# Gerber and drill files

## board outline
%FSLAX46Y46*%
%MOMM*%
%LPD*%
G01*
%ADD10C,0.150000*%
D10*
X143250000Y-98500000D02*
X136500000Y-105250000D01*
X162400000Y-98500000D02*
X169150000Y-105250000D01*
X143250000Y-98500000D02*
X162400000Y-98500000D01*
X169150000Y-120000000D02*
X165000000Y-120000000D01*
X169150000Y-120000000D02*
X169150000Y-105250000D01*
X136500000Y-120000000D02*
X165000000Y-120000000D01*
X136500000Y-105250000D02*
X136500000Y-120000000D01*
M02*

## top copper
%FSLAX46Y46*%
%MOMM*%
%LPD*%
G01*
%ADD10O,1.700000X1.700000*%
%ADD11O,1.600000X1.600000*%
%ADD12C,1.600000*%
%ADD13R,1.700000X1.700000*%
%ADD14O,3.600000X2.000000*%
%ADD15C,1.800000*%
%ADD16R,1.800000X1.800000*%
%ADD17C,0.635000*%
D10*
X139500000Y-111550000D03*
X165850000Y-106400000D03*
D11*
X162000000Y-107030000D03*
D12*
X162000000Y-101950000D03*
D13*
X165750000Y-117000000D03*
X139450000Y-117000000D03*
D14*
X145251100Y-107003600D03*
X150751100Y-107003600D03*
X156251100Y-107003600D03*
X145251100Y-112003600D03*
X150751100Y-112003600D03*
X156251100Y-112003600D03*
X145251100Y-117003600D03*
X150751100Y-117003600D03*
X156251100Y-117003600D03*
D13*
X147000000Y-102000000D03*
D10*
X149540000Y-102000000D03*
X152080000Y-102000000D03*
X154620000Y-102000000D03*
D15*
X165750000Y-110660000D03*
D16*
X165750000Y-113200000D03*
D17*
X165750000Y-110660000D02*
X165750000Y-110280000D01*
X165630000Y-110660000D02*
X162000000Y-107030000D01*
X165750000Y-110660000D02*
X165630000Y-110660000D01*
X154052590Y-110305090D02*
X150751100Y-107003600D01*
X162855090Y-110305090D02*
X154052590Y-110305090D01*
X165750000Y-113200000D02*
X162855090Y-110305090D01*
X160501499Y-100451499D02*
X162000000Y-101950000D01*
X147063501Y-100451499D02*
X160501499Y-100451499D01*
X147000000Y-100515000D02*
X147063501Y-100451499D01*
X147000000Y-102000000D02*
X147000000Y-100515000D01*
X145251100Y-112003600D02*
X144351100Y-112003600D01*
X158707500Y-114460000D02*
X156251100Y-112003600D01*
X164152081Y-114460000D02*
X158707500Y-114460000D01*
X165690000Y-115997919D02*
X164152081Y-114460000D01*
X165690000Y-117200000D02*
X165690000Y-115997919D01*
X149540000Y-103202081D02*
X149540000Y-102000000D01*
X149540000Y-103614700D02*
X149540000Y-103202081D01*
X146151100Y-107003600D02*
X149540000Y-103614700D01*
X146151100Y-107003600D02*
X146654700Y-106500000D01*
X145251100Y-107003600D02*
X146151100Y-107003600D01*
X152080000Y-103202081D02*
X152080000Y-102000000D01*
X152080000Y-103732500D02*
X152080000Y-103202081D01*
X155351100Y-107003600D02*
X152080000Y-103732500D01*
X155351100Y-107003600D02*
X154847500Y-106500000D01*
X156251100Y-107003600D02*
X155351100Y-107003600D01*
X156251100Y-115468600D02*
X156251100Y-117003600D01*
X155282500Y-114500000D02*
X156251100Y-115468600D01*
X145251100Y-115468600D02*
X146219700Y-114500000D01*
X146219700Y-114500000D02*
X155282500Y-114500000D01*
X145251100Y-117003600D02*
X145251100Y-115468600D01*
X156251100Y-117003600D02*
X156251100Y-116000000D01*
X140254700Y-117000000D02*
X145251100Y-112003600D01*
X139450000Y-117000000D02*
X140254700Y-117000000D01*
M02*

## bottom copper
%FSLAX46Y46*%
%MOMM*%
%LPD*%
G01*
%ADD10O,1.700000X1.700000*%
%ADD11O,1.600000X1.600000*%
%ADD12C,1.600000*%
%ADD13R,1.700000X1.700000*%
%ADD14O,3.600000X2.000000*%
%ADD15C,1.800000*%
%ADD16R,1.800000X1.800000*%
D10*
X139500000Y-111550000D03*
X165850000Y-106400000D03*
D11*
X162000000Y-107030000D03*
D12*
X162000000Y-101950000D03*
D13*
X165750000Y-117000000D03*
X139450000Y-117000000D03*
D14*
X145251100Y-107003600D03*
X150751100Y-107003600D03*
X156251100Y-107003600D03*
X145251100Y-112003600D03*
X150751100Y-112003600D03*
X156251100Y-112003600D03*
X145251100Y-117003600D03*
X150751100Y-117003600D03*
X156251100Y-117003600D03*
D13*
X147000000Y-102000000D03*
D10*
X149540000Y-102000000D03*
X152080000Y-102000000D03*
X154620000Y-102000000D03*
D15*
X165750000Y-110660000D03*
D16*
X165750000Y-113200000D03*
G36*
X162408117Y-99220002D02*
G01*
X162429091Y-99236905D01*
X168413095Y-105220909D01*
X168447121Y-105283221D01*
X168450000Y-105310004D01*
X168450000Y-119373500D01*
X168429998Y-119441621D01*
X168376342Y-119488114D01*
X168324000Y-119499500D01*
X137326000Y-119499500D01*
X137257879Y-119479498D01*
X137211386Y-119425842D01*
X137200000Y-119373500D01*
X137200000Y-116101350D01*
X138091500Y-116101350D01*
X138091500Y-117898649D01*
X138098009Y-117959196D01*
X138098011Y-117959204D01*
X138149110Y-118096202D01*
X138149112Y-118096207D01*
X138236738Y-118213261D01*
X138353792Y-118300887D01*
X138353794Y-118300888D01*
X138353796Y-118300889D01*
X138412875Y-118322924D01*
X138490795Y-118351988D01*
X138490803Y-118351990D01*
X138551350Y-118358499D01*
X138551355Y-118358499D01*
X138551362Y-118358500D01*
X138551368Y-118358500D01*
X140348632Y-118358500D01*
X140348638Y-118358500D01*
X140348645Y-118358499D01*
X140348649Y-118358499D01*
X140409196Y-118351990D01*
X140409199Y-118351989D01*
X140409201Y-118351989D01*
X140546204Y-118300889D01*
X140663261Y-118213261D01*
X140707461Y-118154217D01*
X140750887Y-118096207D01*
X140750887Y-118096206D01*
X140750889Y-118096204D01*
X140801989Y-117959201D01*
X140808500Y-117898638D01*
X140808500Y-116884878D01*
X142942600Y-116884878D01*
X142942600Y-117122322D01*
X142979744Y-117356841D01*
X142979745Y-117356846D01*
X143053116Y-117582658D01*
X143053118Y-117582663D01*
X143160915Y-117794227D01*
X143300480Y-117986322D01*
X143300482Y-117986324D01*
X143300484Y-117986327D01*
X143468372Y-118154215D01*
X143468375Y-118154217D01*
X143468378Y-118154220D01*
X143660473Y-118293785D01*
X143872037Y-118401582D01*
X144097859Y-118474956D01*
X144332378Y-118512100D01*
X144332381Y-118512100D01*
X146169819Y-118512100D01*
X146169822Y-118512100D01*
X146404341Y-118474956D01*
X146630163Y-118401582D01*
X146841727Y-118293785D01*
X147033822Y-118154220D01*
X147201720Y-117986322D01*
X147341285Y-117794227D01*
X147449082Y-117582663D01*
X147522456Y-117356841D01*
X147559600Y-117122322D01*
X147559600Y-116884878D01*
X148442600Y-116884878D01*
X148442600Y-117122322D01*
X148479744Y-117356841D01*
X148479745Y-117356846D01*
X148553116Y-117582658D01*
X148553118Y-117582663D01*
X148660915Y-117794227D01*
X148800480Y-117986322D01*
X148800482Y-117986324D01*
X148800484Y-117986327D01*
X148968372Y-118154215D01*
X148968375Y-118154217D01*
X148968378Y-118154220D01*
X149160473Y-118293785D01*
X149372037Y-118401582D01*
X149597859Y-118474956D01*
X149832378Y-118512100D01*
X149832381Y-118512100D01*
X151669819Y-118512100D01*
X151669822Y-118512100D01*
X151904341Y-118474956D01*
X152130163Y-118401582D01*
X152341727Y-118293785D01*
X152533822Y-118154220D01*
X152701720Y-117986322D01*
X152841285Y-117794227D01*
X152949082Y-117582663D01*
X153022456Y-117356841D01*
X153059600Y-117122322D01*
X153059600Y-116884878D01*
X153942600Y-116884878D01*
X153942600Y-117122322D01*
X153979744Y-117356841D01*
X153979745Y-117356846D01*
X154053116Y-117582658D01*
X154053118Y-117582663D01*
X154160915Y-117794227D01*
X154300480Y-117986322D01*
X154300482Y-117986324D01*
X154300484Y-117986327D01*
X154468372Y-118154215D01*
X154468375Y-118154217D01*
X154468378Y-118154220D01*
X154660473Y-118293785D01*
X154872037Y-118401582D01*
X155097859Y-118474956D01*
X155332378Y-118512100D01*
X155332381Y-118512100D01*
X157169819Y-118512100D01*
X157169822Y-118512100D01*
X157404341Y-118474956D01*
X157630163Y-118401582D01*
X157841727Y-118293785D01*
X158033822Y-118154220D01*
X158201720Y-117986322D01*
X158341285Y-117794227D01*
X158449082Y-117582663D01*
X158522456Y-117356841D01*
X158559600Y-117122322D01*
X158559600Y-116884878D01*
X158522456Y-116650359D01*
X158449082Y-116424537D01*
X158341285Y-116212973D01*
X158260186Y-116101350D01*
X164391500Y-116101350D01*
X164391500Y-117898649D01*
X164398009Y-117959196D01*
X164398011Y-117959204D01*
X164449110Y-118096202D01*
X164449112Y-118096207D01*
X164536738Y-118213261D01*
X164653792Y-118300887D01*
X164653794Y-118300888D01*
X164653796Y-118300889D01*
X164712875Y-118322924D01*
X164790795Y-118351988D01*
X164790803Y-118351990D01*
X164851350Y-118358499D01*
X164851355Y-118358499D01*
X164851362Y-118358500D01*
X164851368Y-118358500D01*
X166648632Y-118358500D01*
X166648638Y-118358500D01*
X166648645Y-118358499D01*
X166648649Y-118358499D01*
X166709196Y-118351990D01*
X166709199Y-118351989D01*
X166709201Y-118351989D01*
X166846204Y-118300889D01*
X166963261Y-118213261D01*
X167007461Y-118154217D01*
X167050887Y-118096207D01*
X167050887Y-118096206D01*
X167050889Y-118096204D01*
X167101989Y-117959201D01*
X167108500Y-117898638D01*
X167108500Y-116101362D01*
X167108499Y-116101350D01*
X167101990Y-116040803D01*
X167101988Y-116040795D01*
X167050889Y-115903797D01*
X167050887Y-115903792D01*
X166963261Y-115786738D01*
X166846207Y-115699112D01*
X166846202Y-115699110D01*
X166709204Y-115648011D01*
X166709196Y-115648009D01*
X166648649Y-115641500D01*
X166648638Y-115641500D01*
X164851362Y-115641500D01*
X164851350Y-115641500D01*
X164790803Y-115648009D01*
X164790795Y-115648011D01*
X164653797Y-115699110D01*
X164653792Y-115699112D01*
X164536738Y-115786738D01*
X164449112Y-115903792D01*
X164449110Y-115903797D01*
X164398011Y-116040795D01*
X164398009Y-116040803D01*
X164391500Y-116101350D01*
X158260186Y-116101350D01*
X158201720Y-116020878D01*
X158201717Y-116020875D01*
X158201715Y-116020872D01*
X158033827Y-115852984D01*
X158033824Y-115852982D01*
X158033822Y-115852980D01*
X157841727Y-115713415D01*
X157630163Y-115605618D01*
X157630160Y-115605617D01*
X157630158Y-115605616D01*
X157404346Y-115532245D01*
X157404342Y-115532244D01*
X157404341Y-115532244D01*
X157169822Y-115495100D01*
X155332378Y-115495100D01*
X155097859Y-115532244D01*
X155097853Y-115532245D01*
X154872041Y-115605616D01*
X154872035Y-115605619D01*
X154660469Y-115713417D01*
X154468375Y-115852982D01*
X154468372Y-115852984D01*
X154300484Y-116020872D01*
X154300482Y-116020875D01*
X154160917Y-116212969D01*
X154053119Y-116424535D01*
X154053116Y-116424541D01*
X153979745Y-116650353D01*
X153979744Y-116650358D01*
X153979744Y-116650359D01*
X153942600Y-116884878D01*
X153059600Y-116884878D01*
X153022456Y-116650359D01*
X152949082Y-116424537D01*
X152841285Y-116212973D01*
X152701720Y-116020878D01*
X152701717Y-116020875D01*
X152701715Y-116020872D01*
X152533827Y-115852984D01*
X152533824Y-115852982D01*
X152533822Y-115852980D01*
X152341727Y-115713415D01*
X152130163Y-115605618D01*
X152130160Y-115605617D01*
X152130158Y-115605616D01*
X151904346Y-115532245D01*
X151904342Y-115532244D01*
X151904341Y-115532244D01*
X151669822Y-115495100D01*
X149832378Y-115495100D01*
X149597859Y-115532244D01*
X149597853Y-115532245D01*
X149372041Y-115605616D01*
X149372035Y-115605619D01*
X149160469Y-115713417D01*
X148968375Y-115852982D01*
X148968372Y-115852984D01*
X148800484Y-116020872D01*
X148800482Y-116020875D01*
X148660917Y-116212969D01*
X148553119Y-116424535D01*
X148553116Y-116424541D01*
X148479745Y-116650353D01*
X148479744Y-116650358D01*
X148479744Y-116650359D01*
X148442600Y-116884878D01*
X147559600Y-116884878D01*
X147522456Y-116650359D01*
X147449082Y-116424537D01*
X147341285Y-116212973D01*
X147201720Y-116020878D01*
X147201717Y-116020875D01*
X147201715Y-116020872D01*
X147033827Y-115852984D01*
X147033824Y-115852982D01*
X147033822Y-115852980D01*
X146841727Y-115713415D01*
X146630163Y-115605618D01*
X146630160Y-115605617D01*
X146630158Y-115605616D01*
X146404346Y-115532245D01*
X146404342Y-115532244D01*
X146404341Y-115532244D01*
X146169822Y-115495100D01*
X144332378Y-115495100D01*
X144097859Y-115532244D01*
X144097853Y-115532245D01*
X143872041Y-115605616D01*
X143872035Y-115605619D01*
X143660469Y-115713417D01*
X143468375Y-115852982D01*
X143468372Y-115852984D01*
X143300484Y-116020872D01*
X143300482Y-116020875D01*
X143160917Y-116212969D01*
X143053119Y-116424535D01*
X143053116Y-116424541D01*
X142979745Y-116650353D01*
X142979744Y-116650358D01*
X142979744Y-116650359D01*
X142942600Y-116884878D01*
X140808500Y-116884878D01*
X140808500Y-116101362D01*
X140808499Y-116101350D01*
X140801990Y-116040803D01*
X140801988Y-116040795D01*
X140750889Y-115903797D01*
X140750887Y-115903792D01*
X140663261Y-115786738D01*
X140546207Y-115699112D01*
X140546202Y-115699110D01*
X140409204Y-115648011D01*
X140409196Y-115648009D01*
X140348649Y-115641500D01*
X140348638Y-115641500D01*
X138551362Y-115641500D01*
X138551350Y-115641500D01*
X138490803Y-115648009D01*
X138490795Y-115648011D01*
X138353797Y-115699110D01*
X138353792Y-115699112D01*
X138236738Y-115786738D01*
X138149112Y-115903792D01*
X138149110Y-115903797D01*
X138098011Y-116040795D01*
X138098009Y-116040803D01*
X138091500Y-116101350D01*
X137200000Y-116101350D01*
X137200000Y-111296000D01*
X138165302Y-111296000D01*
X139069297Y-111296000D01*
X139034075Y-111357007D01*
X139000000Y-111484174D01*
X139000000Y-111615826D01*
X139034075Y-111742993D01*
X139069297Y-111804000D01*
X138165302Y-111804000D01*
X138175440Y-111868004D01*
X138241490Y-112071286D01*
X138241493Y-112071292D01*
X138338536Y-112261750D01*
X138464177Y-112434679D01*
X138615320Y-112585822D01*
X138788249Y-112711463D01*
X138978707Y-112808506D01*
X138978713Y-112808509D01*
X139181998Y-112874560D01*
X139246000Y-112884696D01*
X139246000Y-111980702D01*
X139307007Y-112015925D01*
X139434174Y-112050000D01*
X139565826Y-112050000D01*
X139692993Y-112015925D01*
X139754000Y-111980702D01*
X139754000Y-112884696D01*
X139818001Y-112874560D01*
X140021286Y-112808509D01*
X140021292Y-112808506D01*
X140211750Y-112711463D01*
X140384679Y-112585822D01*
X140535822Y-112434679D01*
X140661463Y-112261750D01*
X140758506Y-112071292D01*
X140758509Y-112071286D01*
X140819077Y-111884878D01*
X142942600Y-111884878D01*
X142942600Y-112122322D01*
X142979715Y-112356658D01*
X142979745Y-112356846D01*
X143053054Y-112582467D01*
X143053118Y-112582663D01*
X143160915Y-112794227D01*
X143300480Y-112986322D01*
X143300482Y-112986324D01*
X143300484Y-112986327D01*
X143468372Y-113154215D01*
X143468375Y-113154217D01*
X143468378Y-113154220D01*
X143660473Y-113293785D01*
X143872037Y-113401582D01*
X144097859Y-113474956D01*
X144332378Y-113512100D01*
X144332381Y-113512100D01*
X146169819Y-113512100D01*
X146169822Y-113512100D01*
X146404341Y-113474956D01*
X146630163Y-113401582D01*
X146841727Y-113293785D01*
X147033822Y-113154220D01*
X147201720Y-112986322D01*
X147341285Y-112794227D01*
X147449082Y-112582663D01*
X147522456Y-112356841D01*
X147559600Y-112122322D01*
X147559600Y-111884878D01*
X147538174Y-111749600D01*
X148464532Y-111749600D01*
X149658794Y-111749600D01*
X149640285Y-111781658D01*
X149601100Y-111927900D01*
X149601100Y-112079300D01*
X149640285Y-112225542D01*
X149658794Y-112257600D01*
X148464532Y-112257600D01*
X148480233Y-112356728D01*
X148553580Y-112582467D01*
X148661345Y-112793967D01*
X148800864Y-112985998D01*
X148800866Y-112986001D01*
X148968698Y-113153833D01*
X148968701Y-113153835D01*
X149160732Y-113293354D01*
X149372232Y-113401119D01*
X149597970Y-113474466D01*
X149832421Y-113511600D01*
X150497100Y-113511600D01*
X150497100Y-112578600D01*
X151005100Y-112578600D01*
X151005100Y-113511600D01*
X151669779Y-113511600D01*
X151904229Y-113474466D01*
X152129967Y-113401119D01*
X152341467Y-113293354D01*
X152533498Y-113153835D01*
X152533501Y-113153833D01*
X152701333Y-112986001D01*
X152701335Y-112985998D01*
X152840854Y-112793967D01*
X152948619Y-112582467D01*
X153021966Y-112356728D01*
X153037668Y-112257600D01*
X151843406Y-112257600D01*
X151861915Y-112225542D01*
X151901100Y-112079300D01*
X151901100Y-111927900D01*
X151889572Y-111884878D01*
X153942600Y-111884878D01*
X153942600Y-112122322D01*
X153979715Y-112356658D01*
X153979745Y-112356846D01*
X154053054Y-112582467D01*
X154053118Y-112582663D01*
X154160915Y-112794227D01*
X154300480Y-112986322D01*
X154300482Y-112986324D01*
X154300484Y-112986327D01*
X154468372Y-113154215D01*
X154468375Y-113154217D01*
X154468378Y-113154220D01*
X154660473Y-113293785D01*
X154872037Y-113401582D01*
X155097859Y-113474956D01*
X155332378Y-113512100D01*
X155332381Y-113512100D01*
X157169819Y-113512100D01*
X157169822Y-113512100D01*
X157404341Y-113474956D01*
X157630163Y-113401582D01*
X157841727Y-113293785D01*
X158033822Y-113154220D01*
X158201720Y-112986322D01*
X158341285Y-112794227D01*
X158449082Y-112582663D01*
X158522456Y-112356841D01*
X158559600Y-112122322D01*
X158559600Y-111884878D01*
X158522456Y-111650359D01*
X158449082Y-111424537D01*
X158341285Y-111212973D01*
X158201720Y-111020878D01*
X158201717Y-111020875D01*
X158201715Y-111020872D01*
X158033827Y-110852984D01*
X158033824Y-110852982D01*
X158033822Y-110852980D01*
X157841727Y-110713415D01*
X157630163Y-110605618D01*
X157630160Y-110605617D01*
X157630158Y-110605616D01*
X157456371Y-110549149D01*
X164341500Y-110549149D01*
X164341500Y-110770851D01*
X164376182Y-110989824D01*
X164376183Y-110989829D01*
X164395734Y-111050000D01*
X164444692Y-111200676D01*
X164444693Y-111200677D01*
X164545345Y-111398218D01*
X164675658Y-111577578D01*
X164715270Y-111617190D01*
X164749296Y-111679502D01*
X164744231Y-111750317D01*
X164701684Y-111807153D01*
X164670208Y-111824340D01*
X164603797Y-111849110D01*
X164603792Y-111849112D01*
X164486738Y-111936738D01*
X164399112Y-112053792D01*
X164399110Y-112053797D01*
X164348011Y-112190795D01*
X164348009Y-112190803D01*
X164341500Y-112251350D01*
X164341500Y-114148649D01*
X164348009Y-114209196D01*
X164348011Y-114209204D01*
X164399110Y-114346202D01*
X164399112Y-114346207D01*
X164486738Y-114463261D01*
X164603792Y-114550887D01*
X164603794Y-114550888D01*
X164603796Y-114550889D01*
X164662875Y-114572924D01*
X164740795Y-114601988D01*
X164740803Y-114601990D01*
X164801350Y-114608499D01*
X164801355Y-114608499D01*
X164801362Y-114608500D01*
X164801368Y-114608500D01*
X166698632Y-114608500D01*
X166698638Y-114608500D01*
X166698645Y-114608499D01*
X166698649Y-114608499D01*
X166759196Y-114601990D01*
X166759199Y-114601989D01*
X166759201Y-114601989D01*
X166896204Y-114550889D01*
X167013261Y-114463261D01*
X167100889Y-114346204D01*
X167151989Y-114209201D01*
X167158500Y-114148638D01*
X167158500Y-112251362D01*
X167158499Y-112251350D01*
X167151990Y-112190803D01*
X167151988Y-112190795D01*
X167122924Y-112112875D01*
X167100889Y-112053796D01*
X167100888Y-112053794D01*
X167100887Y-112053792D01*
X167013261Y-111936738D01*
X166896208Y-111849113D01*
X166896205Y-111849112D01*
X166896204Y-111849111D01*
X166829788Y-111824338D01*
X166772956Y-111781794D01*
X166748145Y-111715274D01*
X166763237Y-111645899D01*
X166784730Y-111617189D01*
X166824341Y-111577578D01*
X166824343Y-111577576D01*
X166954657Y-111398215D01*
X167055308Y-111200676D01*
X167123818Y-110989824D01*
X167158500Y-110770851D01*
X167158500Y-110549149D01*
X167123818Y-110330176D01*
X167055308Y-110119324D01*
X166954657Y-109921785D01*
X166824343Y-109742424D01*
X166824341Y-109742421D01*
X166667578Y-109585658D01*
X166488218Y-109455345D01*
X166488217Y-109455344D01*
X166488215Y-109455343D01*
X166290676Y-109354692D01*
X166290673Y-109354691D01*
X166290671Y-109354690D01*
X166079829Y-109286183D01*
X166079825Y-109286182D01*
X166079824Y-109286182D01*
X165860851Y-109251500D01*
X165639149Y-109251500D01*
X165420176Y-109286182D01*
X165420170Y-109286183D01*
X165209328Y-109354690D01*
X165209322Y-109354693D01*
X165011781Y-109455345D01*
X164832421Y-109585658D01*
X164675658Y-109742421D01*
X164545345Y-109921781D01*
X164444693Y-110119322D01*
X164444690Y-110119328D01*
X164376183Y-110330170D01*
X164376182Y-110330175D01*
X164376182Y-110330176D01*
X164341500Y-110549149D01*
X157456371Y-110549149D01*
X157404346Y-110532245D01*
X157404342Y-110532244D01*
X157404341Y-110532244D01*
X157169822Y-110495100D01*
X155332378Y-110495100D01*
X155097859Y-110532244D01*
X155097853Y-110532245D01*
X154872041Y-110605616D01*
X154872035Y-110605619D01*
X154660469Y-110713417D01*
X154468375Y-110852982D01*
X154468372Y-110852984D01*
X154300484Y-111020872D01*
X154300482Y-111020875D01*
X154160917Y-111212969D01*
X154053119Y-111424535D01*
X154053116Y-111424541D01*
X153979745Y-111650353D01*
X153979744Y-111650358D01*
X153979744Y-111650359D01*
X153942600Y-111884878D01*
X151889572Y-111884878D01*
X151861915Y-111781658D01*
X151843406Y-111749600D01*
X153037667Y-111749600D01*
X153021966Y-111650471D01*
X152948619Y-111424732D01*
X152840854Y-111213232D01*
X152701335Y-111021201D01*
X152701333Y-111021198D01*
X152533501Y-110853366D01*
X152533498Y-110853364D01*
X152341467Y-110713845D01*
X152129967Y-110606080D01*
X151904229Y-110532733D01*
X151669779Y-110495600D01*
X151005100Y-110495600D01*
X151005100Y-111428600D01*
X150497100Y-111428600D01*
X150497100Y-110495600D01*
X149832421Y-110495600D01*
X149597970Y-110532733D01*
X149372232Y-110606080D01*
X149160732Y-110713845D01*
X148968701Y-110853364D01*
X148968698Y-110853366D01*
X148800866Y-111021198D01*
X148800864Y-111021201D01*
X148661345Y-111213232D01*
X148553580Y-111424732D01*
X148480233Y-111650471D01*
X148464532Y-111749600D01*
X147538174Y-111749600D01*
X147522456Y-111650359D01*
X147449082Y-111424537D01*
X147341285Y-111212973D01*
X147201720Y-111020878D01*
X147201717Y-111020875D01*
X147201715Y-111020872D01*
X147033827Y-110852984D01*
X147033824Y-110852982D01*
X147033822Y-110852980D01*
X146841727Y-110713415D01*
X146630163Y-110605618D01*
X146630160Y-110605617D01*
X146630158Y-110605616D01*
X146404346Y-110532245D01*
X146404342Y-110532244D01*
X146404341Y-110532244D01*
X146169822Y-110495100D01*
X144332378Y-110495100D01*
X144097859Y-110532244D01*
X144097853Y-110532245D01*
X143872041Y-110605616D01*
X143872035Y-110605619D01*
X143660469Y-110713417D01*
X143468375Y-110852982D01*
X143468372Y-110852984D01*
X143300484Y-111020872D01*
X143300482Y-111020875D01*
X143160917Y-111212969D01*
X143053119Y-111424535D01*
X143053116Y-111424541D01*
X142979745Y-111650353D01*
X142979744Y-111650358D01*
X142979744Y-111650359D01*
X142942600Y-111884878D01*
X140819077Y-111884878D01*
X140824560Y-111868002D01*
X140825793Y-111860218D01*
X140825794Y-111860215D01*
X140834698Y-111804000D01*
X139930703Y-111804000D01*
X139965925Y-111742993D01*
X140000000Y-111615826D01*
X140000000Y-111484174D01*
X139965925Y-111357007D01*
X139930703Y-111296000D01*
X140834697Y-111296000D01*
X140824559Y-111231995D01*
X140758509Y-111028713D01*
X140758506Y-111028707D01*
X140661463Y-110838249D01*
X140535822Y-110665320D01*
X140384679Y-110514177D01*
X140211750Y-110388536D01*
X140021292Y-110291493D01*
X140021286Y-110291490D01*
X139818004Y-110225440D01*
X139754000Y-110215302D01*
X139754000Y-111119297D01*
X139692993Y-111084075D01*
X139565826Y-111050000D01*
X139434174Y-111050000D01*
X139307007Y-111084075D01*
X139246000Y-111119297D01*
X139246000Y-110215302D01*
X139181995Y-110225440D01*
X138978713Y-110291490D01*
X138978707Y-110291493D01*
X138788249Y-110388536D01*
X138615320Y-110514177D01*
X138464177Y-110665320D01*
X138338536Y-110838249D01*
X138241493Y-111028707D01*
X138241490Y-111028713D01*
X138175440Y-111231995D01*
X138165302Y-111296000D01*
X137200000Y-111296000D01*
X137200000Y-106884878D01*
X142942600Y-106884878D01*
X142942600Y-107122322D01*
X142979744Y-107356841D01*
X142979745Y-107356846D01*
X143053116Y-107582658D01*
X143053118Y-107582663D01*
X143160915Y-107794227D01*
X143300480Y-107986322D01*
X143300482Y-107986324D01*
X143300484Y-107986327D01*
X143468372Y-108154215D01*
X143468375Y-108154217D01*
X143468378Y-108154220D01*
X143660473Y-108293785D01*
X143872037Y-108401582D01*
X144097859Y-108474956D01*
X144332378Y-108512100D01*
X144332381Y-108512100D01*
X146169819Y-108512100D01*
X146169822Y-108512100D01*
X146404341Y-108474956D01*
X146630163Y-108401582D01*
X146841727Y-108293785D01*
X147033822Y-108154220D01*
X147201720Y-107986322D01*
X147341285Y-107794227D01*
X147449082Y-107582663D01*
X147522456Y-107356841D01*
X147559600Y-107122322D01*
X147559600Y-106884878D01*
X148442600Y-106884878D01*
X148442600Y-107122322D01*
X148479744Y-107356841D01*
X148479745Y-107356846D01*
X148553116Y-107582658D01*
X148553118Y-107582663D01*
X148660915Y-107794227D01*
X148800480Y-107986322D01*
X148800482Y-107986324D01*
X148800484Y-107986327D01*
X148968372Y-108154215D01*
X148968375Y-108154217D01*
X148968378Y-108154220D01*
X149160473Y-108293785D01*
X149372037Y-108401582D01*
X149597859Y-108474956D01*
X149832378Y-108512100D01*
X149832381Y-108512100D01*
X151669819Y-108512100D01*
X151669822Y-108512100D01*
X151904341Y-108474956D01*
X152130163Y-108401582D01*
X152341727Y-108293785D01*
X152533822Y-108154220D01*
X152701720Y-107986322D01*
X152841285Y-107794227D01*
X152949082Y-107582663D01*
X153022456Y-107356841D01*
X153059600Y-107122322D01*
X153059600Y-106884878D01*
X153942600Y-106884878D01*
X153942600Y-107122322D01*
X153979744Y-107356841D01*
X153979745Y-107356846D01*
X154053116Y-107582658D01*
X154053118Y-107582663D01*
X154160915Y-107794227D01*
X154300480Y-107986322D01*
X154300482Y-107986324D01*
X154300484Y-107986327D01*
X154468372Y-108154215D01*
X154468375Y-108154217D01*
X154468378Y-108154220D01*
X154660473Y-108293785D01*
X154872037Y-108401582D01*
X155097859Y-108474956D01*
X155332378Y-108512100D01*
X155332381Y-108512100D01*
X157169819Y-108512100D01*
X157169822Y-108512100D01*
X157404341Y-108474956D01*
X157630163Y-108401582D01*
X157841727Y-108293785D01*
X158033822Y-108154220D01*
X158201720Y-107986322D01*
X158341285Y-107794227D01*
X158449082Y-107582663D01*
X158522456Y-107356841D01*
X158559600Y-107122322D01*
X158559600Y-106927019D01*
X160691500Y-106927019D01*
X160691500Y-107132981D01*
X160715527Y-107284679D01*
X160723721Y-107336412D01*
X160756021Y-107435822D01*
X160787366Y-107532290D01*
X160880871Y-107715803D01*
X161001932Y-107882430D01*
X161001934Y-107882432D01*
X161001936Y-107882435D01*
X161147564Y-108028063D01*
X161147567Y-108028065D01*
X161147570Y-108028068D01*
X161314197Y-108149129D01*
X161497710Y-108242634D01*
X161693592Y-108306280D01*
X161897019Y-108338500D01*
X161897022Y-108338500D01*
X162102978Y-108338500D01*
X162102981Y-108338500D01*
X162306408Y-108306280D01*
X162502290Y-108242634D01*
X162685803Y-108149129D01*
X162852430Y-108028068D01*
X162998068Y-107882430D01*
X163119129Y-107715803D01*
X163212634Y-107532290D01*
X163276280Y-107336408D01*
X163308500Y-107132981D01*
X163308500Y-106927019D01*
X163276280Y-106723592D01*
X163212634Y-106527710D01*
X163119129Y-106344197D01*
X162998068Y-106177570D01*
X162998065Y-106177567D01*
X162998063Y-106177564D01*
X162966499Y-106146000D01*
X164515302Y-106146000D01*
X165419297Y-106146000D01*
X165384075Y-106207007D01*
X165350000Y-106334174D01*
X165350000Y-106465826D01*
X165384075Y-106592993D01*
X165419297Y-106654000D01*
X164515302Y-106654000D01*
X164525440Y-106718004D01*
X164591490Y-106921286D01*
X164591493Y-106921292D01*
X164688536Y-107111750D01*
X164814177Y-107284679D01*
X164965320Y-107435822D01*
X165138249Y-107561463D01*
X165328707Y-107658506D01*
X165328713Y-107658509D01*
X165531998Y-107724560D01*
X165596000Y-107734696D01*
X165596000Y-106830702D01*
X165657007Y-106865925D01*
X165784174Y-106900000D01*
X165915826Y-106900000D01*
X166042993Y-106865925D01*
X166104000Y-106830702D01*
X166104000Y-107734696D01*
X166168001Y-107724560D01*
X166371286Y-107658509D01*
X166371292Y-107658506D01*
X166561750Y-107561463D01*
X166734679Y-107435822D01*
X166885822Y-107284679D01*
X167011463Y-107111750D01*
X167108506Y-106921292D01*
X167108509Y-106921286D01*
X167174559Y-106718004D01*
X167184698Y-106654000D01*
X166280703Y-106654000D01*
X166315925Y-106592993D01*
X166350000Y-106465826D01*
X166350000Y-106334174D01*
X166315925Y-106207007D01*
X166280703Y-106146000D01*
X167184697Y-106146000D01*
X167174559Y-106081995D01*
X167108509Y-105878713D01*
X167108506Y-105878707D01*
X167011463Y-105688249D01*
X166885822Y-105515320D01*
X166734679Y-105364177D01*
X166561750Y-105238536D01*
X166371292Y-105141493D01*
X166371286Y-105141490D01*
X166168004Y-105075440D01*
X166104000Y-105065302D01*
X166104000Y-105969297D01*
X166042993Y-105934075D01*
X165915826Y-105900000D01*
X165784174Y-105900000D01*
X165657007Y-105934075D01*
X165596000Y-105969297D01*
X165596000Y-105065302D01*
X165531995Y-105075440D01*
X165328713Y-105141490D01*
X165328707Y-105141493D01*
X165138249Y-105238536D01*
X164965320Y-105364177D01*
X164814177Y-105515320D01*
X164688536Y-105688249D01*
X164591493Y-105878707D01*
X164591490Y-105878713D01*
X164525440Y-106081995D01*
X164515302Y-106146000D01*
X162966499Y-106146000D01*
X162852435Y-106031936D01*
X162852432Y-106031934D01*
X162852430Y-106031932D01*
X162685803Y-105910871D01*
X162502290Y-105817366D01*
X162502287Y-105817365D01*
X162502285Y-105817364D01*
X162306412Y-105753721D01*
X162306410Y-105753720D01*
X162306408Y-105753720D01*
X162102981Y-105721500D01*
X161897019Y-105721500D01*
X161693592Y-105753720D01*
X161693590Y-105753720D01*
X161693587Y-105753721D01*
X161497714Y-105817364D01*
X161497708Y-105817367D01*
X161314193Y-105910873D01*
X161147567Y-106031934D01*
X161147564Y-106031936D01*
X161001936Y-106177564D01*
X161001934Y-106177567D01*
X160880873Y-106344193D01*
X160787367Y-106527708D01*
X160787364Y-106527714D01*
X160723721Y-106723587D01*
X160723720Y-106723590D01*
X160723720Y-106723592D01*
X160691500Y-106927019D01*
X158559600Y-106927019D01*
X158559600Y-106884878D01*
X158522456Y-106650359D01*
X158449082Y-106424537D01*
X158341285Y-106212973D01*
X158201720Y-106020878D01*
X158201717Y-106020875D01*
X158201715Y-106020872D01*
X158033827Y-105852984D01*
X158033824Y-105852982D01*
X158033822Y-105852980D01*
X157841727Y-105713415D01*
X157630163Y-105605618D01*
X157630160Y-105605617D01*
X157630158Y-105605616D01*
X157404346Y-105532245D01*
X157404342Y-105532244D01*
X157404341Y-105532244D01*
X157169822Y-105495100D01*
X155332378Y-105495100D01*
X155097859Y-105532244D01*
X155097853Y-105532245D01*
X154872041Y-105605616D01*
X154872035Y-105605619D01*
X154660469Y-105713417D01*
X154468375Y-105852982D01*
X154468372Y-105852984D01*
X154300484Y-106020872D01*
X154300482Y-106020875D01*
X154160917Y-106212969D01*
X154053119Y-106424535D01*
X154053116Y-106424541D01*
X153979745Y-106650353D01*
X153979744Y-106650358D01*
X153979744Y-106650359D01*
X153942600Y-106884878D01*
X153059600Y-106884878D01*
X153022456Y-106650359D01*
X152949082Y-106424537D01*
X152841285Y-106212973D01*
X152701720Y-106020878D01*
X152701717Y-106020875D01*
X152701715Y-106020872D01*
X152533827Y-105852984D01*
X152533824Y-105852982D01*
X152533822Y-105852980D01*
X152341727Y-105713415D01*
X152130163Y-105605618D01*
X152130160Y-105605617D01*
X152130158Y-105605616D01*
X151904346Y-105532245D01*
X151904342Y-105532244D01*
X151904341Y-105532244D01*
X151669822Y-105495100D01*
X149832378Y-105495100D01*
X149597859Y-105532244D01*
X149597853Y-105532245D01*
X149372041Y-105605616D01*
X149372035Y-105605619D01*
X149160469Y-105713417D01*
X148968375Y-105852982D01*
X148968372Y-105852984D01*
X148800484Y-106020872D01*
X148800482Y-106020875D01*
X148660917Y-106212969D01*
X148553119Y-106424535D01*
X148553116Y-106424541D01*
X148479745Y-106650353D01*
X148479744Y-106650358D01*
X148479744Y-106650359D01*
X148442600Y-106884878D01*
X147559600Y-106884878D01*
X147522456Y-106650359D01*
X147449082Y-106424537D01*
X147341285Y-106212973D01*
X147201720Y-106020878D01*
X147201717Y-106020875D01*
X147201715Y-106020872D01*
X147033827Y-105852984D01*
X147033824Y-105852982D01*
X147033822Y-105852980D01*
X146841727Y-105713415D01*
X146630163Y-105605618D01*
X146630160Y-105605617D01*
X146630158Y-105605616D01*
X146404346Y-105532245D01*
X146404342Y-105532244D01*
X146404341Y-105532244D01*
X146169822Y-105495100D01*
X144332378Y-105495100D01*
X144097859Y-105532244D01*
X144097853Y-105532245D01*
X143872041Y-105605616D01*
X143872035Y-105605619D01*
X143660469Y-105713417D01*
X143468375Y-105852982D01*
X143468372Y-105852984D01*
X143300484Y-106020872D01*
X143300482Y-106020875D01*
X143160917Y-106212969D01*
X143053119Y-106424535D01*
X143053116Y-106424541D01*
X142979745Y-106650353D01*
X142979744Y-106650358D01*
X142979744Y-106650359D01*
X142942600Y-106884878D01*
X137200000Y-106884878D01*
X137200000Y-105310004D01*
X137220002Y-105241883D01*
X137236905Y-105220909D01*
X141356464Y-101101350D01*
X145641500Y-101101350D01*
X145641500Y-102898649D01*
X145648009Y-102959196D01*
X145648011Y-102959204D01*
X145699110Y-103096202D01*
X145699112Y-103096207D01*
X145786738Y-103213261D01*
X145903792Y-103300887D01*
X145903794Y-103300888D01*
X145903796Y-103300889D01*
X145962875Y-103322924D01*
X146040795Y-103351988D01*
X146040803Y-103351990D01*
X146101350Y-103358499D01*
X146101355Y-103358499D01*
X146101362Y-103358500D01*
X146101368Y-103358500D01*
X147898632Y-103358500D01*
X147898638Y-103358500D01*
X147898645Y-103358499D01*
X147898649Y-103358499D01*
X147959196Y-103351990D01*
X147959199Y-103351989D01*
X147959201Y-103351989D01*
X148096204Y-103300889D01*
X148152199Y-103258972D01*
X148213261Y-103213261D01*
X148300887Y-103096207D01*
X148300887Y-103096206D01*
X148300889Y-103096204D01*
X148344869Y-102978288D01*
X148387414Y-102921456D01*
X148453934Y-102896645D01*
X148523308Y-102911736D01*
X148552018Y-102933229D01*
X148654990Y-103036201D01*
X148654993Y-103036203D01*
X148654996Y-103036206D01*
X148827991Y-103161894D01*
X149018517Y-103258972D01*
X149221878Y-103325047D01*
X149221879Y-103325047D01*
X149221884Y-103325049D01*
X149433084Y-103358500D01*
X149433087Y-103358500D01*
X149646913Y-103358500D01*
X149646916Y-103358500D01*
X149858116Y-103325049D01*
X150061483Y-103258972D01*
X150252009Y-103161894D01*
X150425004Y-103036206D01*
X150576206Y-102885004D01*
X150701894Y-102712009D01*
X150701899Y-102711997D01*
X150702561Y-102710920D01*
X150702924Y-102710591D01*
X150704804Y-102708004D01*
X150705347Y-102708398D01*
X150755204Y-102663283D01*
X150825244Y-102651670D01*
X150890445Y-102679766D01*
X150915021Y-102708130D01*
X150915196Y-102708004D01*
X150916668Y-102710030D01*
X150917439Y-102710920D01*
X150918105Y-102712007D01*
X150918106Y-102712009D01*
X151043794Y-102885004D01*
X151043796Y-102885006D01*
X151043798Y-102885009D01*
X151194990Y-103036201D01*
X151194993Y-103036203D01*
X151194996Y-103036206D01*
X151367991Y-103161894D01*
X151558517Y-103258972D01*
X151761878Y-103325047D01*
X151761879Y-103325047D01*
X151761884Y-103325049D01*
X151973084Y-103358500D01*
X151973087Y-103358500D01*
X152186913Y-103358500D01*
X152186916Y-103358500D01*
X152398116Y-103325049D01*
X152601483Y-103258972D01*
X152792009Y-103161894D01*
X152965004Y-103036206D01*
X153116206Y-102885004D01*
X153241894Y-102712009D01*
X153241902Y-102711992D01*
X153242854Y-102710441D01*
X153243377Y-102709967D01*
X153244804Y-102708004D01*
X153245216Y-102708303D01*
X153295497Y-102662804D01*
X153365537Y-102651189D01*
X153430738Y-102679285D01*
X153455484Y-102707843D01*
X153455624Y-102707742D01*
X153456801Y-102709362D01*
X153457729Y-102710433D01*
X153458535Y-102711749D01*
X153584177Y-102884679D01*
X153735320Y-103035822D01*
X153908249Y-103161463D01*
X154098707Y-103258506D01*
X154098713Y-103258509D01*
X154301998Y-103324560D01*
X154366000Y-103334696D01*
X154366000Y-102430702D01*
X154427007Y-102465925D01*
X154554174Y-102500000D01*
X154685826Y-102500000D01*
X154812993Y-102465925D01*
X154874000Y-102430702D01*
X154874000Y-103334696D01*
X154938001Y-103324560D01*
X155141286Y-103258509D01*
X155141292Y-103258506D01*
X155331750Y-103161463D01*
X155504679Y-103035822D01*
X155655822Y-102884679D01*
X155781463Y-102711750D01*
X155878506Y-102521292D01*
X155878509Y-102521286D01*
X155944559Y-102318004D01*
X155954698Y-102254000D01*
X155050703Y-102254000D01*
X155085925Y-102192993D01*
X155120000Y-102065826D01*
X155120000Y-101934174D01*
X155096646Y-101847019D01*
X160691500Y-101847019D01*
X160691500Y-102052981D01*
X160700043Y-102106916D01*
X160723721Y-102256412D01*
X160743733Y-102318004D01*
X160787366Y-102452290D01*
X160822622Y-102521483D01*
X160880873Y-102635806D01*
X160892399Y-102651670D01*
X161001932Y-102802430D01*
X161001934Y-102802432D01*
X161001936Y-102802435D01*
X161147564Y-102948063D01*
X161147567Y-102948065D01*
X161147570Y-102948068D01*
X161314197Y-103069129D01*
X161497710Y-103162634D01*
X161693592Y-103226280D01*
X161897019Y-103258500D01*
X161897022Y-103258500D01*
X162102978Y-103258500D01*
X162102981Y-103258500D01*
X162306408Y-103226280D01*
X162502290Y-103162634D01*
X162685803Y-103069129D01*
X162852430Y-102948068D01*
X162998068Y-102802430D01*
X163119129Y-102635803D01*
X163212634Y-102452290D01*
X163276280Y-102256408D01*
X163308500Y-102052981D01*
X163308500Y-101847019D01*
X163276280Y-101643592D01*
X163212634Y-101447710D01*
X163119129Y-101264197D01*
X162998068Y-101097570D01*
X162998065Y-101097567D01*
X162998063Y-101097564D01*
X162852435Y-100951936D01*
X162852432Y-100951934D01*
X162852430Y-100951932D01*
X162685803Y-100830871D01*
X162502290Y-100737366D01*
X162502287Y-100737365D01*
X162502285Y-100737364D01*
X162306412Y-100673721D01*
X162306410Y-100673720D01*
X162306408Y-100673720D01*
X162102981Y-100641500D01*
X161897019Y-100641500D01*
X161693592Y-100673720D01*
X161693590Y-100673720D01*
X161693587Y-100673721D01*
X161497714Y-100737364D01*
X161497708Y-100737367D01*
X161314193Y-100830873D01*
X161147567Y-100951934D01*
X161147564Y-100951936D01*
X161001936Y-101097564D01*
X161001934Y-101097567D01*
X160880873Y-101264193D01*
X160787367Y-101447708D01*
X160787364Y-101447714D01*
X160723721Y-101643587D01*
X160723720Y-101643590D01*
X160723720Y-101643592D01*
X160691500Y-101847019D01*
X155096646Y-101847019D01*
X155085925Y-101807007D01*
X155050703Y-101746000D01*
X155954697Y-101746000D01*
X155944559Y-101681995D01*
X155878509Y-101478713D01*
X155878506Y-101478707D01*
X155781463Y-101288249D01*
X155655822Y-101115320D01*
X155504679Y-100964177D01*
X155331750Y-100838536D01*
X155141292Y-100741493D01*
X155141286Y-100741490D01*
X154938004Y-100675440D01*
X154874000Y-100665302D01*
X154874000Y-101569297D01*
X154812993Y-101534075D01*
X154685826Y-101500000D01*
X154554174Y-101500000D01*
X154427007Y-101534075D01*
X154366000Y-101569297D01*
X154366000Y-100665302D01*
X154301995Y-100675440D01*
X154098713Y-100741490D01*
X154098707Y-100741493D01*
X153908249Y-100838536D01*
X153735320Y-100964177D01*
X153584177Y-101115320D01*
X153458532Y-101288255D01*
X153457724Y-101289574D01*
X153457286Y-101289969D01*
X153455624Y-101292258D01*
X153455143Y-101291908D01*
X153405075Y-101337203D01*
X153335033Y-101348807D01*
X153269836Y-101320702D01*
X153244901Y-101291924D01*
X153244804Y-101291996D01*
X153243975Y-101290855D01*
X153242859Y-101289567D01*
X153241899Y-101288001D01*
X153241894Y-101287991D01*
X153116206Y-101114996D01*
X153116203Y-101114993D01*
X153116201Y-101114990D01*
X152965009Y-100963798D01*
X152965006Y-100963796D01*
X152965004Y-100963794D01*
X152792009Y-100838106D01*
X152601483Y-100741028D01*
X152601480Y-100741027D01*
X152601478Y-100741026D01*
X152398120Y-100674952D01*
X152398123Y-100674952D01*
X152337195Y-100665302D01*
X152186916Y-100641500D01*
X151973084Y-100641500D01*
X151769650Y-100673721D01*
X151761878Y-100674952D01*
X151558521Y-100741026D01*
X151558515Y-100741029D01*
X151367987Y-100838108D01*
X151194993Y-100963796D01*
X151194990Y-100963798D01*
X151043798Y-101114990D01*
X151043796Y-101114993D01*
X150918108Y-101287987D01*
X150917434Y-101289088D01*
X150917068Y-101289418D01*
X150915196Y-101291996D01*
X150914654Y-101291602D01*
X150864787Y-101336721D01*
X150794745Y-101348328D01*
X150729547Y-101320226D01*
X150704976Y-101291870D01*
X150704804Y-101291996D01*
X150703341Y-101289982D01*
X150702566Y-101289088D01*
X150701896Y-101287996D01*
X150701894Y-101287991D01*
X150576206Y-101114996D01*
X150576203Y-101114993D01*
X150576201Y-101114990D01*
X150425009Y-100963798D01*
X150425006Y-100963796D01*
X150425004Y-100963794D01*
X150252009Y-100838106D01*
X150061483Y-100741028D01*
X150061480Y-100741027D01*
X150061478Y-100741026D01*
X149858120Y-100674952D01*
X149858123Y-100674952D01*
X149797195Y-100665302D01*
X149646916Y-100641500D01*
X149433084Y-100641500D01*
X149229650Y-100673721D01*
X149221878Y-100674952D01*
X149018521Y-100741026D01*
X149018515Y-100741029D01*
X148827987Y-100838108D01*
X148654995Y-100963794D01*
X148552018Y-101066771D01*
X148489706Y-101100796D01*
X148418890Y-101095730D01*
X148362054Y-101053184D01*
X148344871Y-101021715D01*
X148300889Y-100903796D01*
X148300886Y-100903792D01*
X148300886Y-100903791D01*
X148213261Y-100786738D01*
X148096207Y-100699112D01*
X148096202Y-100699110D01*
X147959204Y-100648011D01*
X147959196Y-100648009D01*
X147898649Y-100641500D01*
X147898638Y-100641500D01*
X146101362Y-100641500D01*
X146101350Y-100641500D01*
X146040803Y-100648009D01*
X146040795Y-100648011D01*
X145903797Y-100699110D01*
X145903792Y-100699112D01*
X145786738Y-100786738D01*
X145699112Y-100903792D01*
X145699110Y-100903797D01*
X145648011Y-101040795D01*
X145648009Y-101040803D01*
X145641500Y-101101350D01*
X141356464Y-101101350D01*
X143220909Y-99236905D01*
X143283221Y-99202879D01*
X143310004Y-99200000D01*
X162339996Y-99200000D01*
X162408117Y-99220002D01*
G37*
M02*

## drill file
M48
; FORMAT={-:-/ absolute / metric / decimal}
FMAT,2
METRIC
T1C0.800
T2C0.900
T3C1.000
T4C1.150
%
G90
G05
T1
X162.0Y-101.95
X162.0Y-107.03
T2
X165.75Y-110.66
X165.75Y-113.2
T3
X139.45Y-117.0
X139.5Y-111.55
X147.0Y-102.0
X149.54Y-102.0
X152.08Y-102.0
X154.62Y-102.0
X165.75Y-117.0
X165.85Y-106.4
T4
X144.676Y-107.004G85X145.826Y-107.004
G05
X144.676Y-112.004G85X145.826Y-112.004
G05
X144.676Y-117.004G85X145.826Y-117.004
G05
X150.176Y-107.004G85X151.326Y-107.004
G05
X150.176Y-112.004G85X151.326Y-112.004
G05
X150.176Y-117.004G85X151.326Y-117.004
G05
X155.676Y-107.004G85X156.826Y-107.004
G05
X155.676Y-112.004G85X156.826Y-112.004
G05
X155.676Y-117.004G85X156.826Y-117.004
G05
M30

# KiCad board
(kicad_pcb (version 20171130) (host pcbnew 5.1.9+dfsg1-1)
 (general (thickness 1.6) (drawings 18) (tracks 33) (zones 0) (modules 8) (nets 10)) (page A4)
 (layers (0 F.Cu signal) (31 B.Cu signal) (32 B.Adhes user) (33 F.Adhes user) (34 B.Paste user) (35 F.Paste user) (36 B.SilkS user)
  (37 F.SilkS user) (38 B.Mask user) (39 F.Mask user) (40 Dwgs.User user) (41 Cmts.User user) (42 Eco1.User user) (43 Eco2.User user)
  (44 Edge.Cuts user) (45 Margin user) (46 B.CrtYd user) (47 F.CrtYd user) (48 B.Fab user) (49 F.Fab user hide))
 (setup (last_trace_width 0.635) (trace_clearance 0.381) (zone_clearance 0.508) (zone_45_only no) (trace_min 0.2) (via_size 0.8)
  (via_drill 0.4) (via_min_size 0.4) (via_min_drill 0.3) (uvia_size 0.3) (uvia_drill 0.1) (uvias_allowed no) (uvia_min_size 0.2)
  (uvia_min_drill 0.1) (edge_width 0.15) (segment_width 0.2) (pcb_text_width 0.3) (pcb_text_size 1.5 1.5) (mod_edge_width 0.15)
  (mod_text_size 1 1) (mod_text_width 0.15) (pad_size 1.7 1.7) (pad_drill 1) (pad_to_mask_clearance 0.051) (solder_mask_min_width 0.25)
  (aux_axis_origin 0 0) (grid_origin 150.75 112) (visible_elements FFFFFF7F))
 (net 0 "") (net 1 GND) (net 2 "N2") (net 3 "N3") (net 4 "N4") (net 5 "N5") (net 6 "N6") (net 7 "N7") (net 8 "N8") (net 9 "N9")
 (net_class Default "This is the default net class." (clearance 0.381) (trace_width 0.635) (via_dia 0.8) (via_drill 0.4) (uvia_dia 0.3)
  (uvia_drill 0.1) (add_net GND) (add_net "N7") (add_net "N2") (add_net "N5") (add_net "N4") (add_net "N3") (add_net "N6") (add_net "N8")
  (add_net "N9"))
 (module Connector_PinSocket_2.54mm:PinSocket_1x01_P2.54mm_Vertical (layer F.Cu) (at 139.5 111.55)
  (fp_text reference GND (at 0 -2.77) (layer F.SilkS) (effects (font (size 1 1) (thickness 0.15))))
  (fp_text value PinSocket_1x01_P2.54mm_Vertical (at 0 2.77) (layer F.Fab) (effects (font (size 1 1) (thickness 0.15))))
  (pad 1 thru_hole oval (at 0 0) (size 1.7 1.7) (drill 1) (layers *.Cu *.Mask) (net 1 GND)))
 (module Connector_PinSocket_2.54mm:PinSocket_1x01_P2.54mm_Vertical (layer F.Cu) (at 165.85 106.4)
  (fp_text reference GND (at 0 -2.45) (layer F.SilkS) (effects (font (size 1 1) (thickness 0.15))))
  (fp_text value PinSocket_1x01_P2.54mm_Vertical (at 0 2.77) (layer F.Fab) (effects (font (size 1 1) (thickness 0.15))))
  (pad 1 thru_hole oval (at 0 0) (size 1.7 1.7) (drill 1) (layers *.Cu *.Mask) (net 1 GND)))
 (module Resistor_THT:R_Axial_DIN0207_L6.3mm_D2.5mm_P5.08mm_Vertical (layer F.Cu) (at 162 101.95 270)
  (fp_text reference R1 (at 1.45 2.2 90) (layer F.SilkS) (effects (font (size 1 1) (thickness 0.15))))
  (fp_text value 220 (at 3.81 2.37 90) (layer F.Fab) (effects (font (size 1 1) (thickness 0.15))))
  (pad 2 thru_hole oval (at 5.08 0 270) (size 1.6 1.6) (drill 0.8) (layers *.Cu *.Mask) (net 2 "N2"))
  (pad 1 thru_hole circle (at 0 0 270) (size 1.6 1.6) (drill 0.8) (layers *.Cu *.Mask) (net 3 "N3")))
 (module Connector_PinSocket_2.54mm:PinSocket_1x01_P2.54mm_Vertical (layer F.Cu) (at 165.75 117 90)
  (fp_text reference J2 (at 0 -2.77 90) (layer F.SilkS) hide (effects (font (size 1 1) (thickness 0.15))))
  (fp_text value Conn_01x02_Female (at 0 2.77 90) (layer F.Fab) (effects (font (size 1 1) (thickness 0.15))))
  (pad 1 thru_hole rect (at 0 0 90) (size 1.7 1.7) (drill 1) (layers *.Cu *.Mask) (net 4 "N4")))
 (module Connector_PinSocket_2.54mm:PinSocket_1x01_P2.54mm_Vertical (layer F.Cu) (at 139.45 117 180)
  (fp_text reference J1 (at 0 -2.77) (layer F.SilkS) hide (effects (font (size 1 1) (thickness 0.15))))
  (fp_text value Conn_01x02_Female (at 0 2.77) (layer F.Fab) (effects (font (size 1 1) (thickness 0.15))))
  (pad 1 thru_hole rect (at 0 0 180) (size 1.7 1.7) (drill 1) (layers *.Cu *.Mask) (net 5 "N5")))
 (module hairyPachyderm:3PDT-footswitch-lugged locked (layer B.Cu) (at 150.7511 112.0036)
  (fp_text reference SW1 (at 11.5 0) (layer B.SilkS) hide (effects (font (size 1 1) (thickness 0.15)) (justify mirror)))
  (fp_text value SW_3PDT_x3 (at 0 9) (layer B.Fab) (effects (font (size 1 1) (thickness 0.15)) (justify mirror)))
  (pad 3 thru_hole oval (at -5.5 -5 90) (size 2 3.6) (drill oval 1.15 2.3) (layers *.Cu *.Mask) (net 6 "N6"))
  (pad 6 thru_hole oval (at 0 -5 90) (size 2 3.6) (drill oval 1.15 2.3) (layers *.Cu *.Mask) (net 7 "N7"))
  (pad 9 thru_hole oval (at 5.5 -5 90) (size 2 3.6) (drill oval 1.15 2.3) (layers *.Cu *.Mask) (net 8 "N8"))
  (pad 2 thru_hole oval (at -5.5 0 90) (size 2 3.6) (drill oval 1.15 2.3) (layers *.Cu *.Mask) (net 5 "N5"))
  (pad 5 thru_hole oval (at 0 0 90) (size 2 3.6) (drill oval 1.15 2.3) (layers *.Cu *.Mask) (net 1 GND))
  (pad 8 thru_hole oval (at 5.5 0 90) (size 2 3.6) (drill oval 1.15 2.3) (layers *.Cu *.Mask) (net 4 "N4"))
  (pad 1 thru_hole oval (at -5.5 5 90) (size 2 3.6) (drill oval 1.15 2.3) (layers *.Cu *.Mask) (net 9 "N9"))
  (pad 4 thru_hole oval (at 0 5 90) (size 2 3.6) (drill oval 1.15 2.3) (layers *.Cu *.Mask))
  (pad 7 thru_hole oval (at 5.5 5 90) (size 2 3.6) (drill oval 1.15 2.3) (layers *.Cu *.Mask) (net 9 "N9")))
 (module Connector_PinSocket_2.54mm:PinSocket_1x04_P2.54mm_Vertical (layer F.Cu) (at 150.75 102 90)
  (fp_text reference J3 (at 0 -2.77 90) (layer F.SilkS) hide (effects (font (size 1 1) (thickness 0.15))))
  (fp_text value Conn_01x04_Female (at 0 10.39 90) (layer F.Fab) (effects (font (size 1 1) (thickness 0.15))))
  (pad 1 thru_hole rect (at 0 -3.75 90) (size 1.7 1.7) (drill 1) (layers *.Cu *.Mask) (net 3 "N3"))
  (pad 2 thru_hole oval (at 0 -1.21 90) (size 1.7 1.7) (drill 1) (layers *.Cu *.Mask) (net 6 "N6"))
  (pad 3 thru_hole oval (at 0 1.33 90) (size 1.7 1.7) (drill 1) (layers *.Cu *.Mask) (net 8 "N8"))
  (pad 4 thru_hole oval (at 0 3.87 90) (size 1.7 1.7) (drill 1) (layers *.Cu *.Mask) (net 1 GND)))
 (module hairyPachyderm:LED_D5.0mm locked (layer F.Cu) (at 165.75 113.2 90)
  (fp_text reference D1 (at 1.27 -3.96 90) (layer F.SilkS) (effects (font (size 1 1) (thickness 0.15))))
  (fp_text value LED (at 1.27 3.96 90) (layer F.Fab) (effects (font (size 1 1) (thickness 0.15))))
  (pad 2 thru_hole circle (at 2.54 0 90) (size 1.8 1.8) (drill 0.9) (layers *.Cu *.Mask) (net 2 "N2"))
  (pad 1 thru_hole rect (at 0 0 90) (size 1.8 1.8) (drill 0.9) (layers *.Cu *.Mask) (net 7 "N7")))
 (gr_line (start 143.25 98.5) (end 136.5 105.25) (layer Edge.Cuts) (width 0.15))
 (gr_line (start 162.4 98.5) (end 169.15 105.25) (layer Edge.Cuts) (width 0.15))
 (gr_line (start 143.25 98.5) (end 162.4 98.5) (layer Edge.Cuts) (width 0.15))
 (gr_line (start 169.15 120) (end 165 120) (layer Edge.Cuts) (width 0.15))
 (gr_line (start 169.15 120) (end 169.15 105.25) (layer Edge.Cuts) (width 0.15))
 (gr_line (start 136.5 120) (end 165 120) (layer Edge.Cuts) (width 0.15))
 (gr_line (start 136.5 105.25) (end 136.5 120) (layer Edge.Cuts) (width 0.15))
 (segment (start 165.75 110.66) (end 165.75 110.28) (width 0.635) (layer F.Cu) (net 2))
 (segment (start 165.63 110.66) (end 162 107.03) (width 0.635) (layer F.Cu) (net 2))
 (segment (start 165.75 110.66) (end 165.63 110.66) (width 0.635) (layer F.Cu) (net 2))
 (segment (start 154.05259 110.30509) (end 150.7511 107.0036) (width 0.635) (layer F.Cu) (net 7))
 (segment (start 162.85509 110.30509) (end 154.05259 110.30509) (width 0.635) (layer F.Cu) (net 7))
 (segment (start 165.75 113.2) (end 162.85509 110.30509) (width 0.635) (layer F.Cu) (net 7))
 (segment (start 160.501499 100.451499) (end 162 101.95) (width 0.635) (layer F.Cu) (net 3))
 (segment (start 147.063501 100.451499) (end 160.501499 100.451499) (width 0.635) (layer F.Cu) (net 3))
 (segment (start 147 100.515) (end 147.063501 100.451499) (width 0.635) (layer F.Cu) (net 3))
 (segment (start 147 102) (end 147 100.515) (width 0.635) (layer F.Cu) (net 3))
 (segment (start 145.2511 112.0036) (end 144.3511 112.0036) (width 0.635) (layer F.Cu) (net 5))
 (segment (start 158.7075 114.46) (end 156.2511 112.0036) (width 0.635) (layer F.Cu) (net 4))
 (segment (start 164.152081 114.46) (end 158.7075 114.46) (width 0.635) (layer F.Cu) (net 4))
 (segment (start 165.69 115.997919) (end 164.152081 114.46) (width 0.635) (layer F.Cu) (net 4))
 (segment (start 165.69 117.2) (end 165.69 115.997919) (width 0.635) (layer F.Cu) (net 4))
 (segment (start 149.54 103.202081) (end 149.54 102) (width 0.635) (layer F.Cu) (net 6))
 (segment (start 149.54 103.6147) (end 149.54 103.202081) (width 0.635) (layer F.Cu) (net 6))
 (segment (start 146.1511 107.0036) (end 149.54 103.6147) (width 0.635) (layer F.Cu) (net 6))
 (segment (start 146.1511 107.0036) (end 146.6547 106.5) (width 0.635) (layer F.Cu) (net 6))
 (segment (start 145.2511 107.0036) (end 146.1511 107.0036) (width 0.635) (layer F.Cu) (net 6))
 (segment (start 152.08 103.202081) (end 152.08 102) (width 0.635) (layer F.Cu) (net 8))
 (segment (start 152.08 103.7325) (end 152.08 103.202081) (width 0.635) (layer F.Cu) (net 8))
 (segment (start 155.3511 107.0036) (end 152.08 103.7325) (width 0.635) (layer F.Cu) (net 8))
 (segment (start 155.3511 107.0036) (end 154.8475 106.5) (width 0.635) (layer F.Cu) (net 8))
 (segment (start 156.2511 107.0036) (end 155.3511 107.0036) (width 0.635) (layer F.Cu) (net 8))
 (segment (start 156.2511 115.4686) (end 156.2511 117.0036) (width 0.635) (layer F.Cu) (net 9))
 (segment (start 155.2825 114.5) (end 156.2511 115.4686) (width 0.635) (layer F.Cu) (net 9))
 (segment (start 145.2511 115.4686) (end 146.2197 114.5) (width 0.635) (layer F.Cu) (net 9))
 (segment (start 146.2197 114.5) (end 155.2825 114.5) (width 0.635) (layer F.Cu) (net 9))
 (segment (start 145.2511 117.0036) (end 145.2511 115.4686) (width 0.635) (layer F.Cu) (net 9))
 (segment (start 156.2511 117.0036) (end 156.2511 116) (width 0.635) (layer F.Cu) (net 9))
 (segment (start 140.2547 117) (end 145.2511 112.0036) (width 0.635) (layer F.Cu) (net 5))
 (segment (start 139.45 117) (end 140.2547 117) (width 0.635) (layer F.Cu) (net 5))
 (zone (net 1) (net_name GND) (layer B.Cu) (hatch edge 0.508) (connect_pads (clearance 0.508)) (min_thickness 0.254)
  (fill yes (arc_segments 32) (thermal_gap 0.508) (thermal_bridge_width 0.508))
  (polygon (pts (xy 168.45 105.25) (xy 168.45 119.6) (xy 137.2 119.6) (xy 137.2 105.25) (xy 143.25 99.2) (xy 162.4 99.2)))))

